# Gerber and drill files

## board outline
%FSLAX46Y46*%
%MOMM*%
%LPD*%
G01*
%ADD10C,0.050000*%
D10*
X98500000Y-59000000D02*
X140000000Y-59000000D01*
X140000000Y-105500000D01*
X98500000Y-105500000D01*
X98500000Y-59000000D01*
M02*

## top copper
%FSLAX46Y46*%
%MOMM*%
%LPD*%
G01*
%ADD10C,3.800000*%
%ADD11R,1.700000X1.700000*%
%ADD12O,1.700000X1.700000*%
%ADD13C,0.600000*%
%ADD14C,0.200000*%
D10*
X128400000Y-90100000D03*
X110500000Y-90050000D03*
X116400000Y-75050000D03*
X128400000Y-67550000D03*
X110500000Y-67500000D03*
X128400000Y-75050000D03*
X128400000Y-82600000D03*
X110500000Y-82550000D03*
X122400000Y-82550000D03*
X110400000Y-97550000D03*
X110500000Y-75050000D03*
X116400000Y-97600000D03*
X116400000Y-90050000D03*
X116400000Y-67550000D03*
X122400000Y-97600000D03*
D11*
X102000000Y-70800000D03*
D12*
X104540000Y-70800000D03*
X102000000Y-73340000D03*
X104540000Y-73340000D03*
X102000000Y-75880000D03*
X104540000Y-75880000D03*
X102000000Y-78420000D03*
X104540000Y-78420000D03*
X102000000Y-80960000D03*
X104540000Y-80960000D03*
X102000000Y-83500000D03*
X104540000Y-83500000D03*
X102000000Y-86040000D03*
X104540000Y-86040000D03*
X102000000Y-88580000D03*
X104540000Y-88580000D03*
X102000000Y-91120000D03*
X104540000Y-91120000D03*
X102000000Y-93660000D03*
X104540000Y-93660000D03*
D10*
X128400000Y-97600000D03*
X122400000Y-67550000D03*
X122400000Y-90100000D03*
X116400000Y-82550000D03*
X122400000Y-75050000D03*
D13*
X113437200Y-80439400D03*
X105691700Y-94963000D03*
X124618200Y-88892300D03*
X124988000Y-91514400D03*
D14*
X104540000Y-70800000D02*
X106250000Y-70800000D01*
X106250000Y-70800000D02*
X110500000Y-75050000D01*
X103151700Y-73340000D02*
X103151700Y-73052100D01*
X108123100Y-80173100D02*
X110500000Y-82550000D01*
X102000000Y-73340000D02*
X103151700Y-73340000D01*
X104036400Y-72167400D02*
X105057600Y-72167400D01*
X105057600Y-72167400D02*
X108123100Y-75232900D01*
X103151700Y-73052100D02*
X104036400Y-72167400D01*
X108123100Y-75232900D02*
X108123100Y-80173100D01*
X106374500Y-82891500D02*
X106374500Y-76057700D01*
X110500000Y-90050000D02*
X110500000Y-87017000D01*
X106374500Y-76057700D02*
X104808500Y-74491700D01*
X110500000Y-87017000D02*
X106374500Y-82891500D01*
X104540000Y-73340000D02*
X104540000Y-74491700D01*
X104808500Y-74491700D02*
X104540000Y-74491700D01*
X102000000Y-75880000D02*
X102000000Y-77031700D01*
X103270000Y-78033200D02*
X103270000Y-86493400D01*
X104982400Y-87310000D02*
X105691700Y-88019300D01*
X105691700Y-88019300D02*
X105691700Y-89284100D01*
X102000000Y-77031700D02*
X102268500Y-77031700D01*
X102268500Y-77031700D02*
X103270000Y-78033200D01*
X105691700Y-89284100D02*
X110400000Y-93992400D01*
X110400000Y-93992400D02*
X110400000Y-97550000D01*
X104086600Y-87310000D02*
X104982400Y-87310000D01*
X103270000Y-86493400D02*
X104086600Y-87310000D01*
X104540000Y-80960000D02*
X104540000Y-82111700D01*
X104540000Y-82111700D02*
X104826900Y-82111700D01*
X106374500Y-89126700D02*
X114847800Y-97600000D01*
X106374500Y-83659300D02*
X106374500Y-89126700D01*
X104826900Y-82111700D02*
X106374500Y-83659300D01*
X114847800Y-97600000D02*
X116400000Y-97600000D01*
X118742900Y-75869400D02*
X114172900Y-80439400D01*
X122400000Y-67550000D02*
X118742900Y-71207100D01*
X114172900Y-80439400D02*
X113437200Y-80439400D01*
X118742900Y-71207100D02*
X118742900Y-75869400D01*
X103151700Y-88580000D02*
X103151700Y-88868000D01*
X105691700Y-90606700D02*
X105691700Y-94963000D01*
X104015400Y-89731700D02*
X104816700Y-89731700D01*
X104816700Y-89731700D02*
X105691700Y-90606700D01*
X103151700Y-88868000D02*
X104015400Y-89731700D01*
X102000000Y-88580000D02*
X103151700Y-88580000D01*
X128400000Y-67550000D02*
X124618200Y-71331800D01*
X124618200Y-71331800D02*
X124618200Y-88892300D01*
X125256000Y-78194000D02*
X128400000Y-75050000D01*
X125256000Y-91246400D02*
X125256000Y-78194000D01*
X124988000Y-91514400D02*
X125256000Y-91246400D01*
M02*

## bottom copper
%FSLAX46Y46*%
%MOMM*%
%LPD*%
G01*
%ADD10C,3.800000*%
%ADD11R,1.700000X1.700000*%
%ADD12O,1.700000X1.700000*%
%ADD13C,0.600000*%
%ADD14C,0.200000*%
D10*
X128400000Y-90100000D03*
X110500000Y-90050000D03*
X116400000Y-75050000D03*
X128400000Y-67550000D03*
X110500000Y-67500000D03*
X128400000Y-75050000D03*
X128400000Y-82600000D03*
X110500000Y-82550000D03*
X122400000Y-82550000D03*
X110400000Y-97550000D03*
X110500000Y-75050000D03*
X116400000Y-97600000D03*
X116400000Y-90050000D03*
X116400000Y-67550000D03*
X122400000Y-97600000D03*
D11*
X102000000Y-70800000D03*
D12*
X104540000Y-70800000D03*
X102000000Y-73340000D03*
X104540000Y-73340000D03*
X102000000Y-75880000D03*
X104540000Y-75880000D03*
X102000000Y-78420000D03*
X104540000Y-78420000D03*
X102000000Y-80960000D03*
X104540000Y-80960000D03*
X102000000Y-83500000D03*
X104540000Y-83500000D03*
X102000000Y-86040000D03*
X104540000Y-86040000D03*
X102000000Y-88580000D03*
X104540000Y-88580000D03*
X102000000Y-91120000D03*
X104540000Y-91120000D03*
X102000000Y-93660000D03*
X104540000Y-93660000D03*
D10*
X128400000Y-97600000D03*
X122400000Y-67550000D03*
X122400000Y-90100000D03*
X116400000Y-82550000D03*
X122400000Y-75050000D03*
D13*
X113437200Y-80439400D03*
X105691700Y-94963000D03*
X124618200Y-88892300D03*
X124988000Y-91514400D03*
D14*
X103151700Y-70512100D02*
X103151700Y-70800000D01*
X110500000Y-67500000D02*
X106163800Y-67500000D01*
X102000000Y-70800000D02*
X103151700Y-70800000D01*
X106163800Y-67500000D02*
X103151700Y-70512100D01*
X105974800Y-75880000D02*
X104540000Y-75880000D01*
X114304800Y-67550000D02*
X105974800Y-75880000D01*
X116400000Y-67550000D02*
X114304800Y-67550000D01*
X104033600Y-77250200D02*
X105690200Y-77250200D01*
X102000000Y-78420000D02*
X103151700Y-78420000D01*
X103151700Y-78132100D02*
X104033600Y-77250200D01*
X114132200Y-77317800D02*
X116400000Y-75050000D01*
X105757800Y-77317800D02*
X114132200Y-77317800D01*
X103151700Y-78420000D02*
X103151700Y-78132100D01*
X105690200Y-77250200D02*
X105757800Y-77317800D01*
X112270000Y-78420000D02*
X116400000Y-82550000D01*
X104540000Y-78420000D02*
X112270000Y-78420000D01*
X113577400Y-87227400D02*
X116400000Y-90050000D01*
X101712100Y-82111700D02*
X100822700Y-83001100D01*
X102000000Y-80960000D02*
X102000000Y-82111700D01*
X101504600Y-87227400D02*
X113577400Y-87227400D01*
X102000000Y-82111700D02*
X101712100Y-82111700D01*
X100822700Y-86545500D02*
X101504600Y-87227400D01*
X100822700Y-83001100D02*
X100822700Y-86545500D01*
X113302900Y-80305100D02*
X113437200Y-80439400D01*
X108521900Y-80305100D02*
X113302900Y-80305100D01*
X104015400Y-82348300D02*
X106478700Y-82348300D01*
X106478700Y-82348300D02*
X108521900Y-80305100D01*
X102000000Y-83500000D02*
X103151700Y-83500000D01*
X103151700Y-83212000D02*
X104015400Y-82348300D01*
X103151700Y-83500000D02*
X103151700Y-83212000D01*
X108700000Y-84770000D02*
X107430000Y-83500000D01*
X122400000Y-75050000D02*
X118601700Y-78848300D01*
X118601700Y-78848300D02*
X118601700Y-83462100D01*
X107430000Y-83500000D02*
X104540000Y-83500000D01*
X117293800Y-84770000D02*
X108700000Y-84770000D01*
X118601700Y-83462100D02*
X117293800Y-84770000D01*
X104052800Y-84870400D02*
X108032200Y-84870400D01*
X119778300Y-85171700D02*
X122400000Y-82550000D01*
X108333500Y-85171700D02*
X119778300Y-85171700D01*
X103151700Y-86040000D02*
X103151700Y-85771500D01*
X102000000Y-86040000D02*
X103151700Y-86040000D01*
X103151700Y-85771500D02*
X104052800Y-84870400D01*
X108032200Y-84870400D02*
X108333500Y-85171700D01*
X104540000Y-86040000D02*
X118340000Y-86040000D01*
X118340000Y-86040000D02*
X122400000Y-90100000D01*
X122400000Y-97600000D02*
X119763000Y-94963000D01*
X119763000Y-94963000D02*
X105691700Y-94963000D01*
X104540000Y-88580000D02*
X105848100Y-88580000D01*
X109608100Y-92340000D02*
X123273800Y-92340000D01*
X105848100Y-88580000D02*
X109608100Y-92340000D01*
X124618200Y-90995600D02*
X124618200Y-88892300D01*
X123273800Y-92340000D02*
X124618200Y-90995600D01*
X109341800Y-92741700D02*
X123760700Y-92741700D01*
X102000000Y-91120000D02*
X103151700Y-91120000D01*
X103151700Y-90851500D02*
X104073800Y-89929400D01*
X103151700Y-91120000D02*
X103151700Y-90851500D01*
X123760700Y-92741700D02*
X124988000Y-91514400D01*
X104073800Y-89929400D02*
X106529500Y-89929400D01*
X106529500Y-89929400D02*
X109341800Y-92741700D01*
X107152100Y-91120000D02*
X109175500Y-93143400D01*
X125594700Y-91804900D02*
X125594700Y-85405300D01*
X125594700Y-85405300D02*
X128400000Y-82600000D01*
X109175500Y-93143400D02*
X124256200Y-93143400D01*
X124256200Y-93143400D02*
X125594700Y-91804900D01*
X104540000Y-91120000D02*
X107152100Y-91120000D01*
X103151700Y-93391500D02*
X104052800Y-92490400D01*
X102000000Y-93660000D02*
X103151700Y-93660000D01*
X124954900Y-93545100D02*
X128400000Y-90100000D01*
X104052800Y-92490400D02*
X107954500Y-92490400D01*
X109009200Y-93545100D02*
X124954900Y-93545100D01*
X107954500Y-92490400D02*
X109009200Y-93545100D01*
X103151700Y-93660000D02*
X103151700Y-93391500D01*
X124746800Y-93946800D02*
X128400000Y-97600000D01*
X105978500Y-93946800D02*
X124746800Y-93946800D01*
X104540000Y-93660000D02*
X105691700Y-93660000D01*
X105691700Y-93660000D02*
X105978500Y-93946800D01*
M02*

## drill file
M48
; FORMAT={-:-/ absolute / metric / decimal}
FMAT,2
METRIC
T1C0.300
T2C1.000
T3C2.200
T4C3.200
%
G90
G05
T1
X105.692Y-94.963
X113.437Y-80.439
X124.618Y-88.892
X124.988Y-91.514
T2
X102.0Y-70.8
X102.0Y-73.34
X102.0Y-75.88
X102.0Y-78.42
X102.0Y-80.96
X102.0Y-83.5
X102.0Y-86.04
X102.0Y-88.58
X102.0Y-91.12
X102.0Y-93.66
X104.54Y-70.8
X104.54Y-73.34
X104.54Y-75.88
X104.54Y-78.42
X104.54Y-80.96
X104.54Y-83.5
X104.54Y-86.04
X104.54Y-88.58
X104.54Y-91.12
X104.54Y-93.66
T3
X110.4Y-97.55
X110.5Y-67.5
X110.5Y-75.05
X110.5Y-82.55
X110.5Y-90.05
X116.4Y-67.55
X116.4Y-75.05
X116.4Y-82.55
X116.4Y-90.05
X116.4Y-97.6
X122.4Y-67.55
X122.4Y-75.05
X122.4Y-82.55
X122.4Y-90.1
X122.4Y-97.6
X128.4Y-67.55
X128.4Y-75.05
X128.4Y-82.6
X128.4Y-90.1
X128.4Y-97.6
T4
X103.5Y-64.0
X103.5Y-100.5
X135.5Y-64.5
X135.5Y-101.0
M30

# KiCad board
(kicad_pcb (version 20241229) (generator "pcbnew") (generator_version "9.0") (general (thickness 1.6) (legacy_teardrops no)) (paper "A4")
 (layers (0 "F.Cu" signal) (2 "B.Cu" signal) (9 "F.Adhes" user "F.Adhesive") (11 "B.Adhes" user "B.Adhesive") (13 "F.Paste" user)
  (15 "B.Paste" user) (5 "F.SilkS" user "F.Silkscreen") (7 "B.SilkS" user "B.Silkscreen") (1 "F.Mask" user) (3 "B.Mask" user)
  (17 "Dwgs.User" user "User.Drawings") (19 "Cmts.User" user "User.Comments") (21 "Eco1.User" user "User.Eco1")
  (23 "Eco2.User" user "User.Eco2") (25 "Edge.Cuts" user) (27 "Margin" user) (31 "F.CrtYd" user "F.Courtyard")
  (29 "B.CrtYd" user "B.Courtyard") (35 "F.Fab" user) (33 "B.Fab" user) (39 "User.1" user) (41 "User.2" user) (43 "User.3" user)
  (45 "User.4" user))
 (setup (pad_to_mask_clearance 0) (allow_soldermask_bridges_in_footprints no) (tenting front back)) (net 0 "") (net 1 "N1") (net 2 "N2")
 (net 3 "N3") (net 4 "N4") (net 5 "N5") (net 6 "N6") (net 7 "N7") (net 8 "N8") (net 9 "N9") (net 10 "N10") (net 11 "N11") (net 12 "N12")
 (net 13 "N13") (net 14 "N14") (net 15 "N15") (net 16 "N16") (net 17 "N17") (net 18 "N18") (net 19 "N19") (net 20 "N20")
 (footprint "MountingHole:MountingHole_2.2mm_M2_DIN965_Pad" (layer "F.Cu") (at 128.4 90.1)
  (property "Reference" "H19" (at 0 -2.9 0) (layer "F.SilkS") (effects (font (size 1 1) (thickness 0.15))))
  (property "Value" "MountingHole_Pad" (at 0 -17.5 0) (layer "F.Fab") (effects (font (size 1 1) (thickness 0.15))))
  (pad "1" thru_hole circle (at 0 0) (size 3.8 3.8) (drill 2.2) (layers "*.Cu" "*.Mask") (remove_unused_layers no) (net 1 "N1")))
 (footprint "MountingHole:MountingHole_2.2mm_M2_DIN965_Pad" (layer "F.Cu") (at 110.5 90.05)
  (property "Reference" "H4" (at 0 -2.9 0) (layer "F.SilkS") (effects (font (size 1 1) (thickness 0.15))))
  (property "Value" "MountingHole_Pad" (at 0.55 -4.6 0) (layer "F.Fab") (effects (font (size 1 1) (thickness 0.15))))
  (pad "1" thru_hole circle (at 0 0) (size 3.8 3.8) (drill 2.2) (layers "*.Cu" "*.Mask") (remove_unused_layers no) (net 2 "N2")))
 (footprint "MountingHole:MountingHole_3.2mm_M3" (layer "F.Cu") (at 135.5 64.5)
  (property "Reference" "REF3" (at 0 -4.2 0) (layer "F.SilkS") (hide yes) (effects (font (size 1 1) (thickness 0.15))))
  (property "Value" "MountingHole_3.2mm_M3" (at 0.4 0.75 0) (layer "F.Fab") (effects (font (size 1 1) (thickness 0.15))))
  (pad "" np_thru_hole circle (at 0 0) (size 3.2 3.2) (drill 3.2) (layers "*.Cu" "*.Mask")))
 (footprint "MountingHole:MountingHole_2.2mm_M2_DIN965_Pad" (layer "F.Cu") (at 116.4 75.05)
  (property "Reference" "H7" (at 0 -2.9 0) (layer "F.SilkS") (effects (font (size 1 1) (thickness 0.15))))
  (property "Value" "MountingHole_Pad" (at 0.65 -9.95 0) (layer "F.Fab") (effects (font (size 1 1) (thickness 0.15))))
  (pad "1" thru_hole circle (at 0 0) (size 3.8 3.8) (drill 2.2) (layers "*.Cu" "*.Mask") (remove_unused_layers no) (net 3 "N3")))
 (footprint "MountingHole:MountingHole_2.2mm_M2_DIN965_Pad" (layer "F.Cu") (at 128.4 67.55)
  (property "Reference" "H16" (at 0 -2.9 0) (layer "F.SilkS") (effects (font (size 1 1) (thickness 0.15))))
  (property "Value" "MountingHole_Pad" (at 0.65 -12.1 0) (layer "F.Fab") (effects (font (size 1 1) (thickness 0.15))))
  (pad "1" thru_hole circle (at 0 0) (size 3.8 3.8) (drill 2.2) (layers "*.Cu" "*.Mask") (remove_unused_layers no) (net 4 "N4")))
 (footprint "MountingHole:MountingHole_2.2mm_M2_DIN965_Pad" (layer "F.Cu") (at 110.5 67.5)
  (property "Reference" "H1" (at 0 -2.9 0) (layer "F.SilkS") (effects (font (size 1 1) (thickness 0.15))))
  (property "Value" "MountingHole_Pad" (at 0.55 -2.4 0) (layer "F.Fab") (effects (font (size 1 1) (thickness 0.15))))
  (pad "1" thru_hole circle (at 0 0) (size 3.8 3.8) (drill 2.2) (layers "*.Cu" "*.Mask") (remove_unused_layers no) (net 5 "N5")))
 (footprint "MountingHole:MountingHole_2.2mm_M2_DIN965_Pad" (layer "F.Cu") (at 128.4 75.05)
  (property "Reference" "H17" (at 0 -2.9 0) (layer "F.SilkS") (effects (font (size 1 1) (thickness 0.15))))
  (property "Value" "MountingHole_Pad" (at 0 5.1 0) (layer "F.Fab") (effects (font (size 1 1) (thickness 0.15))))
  (pad "1" thru_hole circle (at 0 0) (size 3.8 3.8) (drill 2.2) (layers "*.Cu" "*.Mask") (remove_unused_layers no) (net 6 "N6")))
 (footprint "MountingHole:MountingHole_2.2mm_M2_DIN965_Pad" (layer "F.Cu") (at 128.4 82.6)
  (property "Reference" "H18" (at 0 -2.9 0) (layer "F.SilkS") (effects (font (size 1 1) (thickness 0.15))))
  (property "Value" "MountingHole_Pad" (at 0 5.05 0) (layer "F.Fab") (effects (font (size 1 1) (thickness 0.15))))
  (pad "1" thru_hole circle (at 0 0) (size 3.8 3.8) (drill 2.2) (layers "*.Cu" "*.Mask") (remove_unused_layers no) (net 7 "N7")))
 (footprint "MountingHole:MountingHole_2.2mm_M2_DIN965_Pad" (layer "F.Cu") (at 110.5 82.55)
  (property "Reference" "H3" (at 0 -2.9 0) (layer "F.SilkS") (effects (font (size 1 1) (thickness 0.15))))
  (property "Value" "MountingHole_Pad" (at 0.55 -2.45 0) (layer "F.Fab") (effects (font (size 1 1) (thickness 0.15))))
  (pad "1" thru_hole circle (at 0 0) (size 3.8 3.8) (drill 2.2) (layers "*.Cu" "*.Mask") (remove_unused_layers no) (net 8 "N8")))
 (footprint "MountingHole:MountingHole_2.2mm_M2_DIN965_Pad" (layer "F.Cu") (at 122.4 82.55)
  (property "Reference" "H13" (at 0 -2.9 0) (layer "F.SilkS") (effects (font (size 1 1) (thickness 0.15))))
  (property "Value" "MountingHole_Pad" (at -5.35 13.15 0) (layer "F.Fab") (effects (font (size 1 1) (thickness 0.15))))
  (pad "1" thru_hole circle (at 0 0) (size 3.8 3.8) (drill 2.2) (layers "*.Cu" "*.Mask") (remove_unused_layers no) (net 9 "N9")))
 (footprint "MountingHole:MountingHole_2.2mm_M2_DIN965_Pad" (layer "F.Cu") (at 110.4 97.55)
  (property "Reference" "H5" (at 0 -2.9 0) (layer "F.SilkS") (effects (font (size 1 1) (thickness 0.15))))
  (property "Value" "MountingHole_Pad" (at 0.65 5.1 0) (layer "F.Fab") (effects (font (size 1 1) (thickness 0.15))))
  (pad "1" thru_hole circle (at 0 0) (size 3.8 3.8) (drill 2.2) (layers "*.Cu" "*.Mask") (remove_unused_layers no) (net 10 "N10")))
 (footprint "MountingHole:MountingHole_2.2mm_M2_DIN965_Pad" (layer "F.Cu") (at 110.5 75.05)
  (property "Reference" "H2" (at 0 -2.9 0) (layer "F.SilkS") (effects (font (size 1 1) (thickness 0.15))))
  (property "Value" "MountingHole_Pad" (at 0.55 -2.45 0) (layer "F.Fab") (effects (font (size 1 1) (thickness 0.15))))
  (pad "1" thru_hole circle (at 0 0) (size 3.8 3.8) (drill 2.2) (layers "*.Cu" "*.Mask") (remove_unused_layers no) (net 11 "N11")))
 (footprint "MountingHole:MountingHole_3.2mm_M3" (layer "F.Cu") (at 135.5 101)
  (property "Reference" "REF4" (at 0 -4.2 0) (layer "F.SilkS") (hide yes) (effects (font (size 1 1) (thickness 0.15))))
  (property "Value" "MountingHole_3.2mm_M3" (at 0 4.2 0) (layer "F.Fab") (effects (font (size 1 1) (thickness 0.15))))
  (pad "" np_thru_hole circle (at 0 0) (size 3.2 3.2) (drill 3.2) (layers "*.Cu" "*.Mask")))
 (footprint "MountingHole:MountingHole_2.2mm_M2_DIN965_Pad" (layer "F.Cu") (at 116.4 97.6)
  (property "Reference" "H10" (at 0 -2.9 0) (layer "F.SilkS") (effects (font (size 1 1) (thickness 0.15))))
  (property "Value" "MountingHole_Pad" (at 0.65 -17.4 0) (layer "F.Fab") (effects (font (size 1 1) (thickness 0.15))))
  (pad "1" thru_hole circle (at 0 0) (size 3.8 3.8) (drill 2.2) (layers "*.Cu" "*.Mask") (remove_unused_layers no) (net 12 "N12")))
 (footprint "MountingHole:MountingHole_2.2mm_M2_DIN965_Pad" (layer "F.Cu") (at 116.4 90.05)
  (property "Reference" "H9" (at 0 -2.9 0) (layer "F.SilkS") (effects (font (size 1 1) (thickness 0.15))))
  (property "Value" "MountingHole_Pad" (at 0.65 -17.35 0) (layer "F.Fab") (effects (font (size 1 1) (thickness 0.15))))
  (pad "1" thru_hole circle (at 0 0) (size 3.8 3.8) (drill 2.2) (layers "*.Cu" "*.Mask") (remove_unused_layers no) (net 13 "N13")))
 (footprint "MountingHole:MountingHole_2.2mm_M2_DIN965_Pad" (layer "F.Cu") (at 116.4 67.55)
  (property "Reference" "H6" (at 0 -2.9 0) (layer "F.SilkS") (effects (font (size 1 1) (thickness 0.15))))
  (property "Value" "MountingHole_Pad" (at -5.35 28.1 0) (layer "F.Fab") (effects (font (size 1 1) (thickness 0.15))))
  (pad "1" thru_hole circle (at 0 0) (size 3.8 3.8) (drill 2.2) (layers "*.Cu" "*.Mask") (remove_unused_layers no) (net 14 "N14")))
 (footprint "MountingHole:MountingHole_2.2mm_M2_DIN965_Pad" (layer "F.Cu") (at 122.4 97.6)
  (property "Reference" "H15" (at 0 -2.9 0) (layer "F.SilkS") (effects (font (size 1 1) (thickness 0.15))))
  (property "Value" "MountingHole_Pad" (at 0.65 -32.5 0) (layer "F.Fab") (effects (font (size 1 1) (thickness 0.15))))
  (pad "1" thru_hole circle (at 0 0) (size 3.8 3.8) (drill 2.2) (layers "*.Cu" "*.Mask") (remove_unused_layers no) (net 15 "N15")))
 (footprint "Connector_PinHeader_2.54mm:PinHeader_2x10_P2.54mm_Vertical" (layer "F.Cu") (at 102 70.8)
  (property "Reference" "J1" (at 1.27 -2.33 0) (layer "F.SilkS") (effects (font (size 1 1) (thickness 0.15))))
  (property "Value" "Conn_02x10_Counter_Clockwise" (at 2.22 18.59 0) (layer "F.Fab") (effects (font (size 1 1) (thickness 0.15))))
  (pad "1" thru_hole rect (at 0 0) (size 1.7 1.7) (drill 1) (layers "*.Cu" "*.Mask") (remove_unused_layers no) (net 5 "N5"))
  (pad "2" thru_hole oval (at 2.54 0) (size 1.7 1.7) (drill 1) (layers "*.Cu" "*.Mask") (remove_unused_layers no) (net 11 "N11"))
  (pad "3" thru_hole oval (at 0 2.54) (size 1.7 1.7) (drill 1) (layers "*.Cu" "*.Mask") (remove_unused_layers no) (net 8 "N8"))
  (pad "4" thru_hole oval (at 2.54 2.54) (size 1.7 1.7) (drill 1) (layers "*.Cu" "*.Mask") (remove_unused_layers no) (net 2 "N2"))
  (pad "5" thru_hole oval (at 0 5.08) (size 1.7 1.7) (drill 1) (layers "*.Cu" "*.Mask") (remove_unused_layers no) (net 10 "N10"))
  (pad "6" thru_hole oval (at 2.54 5.08) (size 1.7 1.7) (drill 1) (layers "*.Cu" "*.Mask") (remove_unused_layers no) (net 14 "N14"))
  (pad "7" thru_hole oval (at 0 7.62) (size 1.7 1.7) (drill 1) (layers "*.Cu" "*.Mask") (remove_unused_layers no) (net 3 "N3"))
  (pad "8" thru_hole oval (at 2.54 7.62) (size 1.7 1.7) (drill 1) (layers "*.Cu" "*.Mask") (remove_unused_layers no) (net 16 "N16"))
  (pad "9" thru_hole oval (at 0 10.16) (size 1.7 1.7) (drill 1) (layers "*.Cu" "*.Mask") (remove_unused_layers no) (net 13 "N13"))
  (pad "10" thru_hole oval (at 2.54 10.16) (size 1.7 1.7) (drill 1) (layers "*.Cu" "*.Mask") (remove_unused_layers no) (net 12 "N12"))
  (pad "11" thru_hole oval (at 0 12.7) (size 1.7 1.7) (drill 1) (layers "*.Cu" "*.Mask") (remove_unused_layers no) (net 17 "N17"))
  (pad "12" thru_hole oval (at 2.54 12.7) (size 1.7 1.7) (drill 1) (layers "*.Cu" "*.Mask") (remove_unused_layers no) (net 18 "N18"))
  (pad "13" thru_hole oval (at 0 15.24) (size 1.7 1.7) (drill 1) (layers "*.Cu" "*.Mask") (remove_unused_layers no) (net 9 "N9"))
  (pad "14" thru_hole oval (at 2.54 15.24) (size 1.7 1.7) (drill 1) (layers "*.Cu" "*.Mask") (remove_unused_layers no) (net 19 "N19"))
  (pad "15" thru_hole oval (at 0 17.78) (size 1.7 1.7) (drill 1) (layers "*.Cu" "*.Mask") (remove_unused_layers no) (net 15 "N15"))
  (pad "16" thru_hole oval (at 2.54 17.78) (size 1.7 1.7) (drill 1) (layers "*.Cu" "*.Mask") (remove_unused_layers no) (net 4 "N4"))
  (pad "17" thru_hole oval (at 0 20.32) (size 1.7 1.7) (drill 1) (layers "*.Cu" "*.Mask") (remove_unused_layers no) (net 6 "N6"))
  (pad "18" thru_hole oval (at 2.54 20.32) (size 1.7 1.7) (drill 1) (layers "*.Cu" "*.Mask") (remove_unused_layers no) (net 7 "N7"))
  (pad "19" thru_hole oval (at 0 22.86) (size 1.7 1.7) (drill 1) (layers "*.Cu" "*.Mask") (remove_unused_layers no) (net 1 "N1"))
  (pad "20" thru_hole oval (at 2.54 22.86) (size 1.7 1.7) (drill 1) (layers "*.Cu" "*.Mask") (remove_unused_layers no) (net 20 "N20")))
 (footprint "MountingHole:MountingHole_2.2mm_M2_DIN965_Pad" (layer "F.Cu") (at 128.4 97.6)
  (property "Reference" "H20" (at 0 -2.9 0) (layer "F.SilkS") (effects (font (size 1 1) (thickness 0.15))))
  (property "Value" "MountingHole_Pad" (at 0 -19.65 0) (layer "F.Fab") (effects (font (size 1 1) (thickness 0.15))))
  (pad "1" thru_hole circle (at 0 0) (size 3.8 3.8) (drill 2.2) (layers "*.Cu" "*.Mask") (remove_unused_layers no) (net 20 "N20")))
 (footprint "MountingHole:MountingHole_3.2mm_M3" (layer "F.Cu") (at 103.5 100.5)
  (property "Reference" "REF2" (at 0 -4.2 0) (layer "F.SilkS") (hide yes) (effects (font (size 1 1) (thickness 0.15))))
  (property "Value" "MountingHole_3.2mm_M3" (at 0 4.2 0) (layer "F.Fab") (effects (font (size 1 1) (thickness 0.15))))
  (pad "" np_thru_hole circle (at 0 0) (size 3.2 3.2) (drill 3.2) (layers "*.Cu" "*.Mask")))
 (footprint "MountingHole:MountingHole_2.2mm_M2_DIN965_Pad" (layer "F.Cu") (at 122.4 67.55)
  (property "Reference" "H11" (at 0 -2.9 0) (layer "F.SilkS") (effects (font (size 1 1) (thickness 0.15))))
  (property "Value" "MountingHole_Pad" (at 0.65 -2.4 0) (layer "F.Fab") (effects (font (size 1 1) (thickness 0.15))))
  (pad "1" thru_hole circle (at 0 0) (size 3.8 3.8) (drill 2.2) (layers "*.Cu" "*.Mask") (remove_unused_layers no) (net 17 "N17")))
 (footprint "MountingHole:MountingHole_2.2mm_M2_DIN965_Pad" (layer "F.Cu") (at 122.4 90.1)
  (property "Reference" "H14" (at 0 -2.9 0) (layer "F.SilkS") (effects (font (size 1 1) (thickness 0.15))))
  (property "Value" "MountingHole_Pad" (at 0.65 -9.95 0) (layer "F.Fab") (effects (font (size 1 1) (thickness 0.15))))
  (pad "1" thru_hole circle (at 0 0) (size 3.8 3.8) (drill 2.2) (layers "*.Cu" "*.Mask") (remove_unused_layers no) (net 19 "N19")))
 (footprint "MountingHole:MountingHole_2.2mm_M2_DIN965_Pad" (layer "F.Cu") (at 116.4 82.55)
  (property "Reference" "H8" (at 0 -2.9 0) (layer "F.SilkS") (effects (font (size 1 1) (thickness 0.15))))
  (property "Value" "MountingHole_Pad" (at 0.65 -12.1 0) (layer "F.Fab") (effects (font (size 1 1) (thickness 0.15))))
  (pad "1" thru_hole circle (at 0 0) (size 3.8 3.8) (drill 2.2) (layers "*.Cu" "*.Mask") (remove_unused_layers no) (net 16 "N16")))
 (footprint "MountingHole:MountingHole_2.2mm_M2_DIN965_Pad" (layer "F.Cu") (at 122.4 75.05)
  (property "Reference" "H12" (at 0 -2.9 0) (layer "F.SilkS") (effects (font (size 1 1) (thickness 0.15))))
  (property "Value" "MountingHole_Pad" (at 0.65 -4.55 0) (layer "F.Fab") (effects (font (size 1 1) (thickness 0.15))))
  (pad "1" thru_hole circle (at 0 0) (size 3.8 3.8) (drill 2.2) (layers "*.Cu" "*.Mask") (remove_unused_layers no) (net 18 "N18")))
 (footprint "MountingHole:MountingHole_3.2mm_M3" (layer "F.Cu") (at 103.5 64)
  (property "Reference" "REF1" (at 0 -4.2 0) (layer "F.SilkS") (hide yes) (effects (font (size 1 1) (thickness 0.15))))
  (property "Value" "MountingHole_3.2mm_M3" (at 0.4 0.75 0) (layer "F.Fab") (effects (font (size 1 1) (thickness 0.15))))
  (pad "" np_thru_hole circle (at 0 0) (size 3.2 3.2) (drill 3.2) (layers "*.Cu" "*.Mask")))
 (gr_rect (start 98.5 59) (end 140 105.5) (stroke (width 0.05) (type default)) (fill no) (layer "Edge.Cuts"))
 (segment (start 103.1517 70.5121) (end 103.1517 70.8) (width 0.2) (layer "B.Cu") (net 5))
 (segment (start 110.5 67.5) (end 106.1638 67.5) (width 0.2) (layer "B.Cu") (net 5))
 (segment (start 102 70.8) (end 103.1517 70.8) (width 0.2) (layer "B.Cu") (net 5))
 (segment (start 106.1638 67.5) (end 103.1517 70.5121) (width 0.2) (layer "B.Cu") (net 5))
 (segment (start 104.54 70.8) (end 106.25 70.8) (width 0.2) (layer "F.Cu") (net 11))
 (segment (start 106.25 70.8) (end 110.5 75.05) (width 0.2) (layer "F.Cu") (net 11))
 (segment (start 103.1517 73.34) (end 103.1517 73.0521) (width 0.2) (layer "F.Cu") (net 8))
 (segment (start 108.1231 80.1731) (end 110.5 82.55) (width 0.2) (layer "F.Cu") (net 8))
 (segment (start 102 73.34) (end 103.1517 73.34) (width 0.2) (layer "F.Cu") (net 8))
 (segment (start 104.0364 72.1674) (end 105.0576 72.1674) (width 0.2) (layer "F.Cu") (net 8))
 (segment (start 105.0576 72.1674) (end 108.1231 75.2329) (width 0.2) (layer "F.Cu") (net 8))
 (segment (start 103.1517 73.0521) (end 104.0364 72.1674) (width 0.2) (layer "F.Cu") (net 8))
 (segment (start 108.1231 75.2329) (end 108.1231 80.1731) (width 0.2) (layer "F.Cu") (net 8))
 (segment (start 106.3745 82.8915) (end 106.3745 76.0577) (width 0.2) (layer "F.Cu") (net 2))
 (segment (start 110.5 90.05) (end 110.5 87.017) (width 0.2) (layer "F.Cu") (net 2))
 (segment (start 106.3745 76.0577) (end 104.8085 74.4917) (width 0.2) (layer "F.Cu") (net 2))
 (segment (start 110.5 87.017) (end 106.3745 82.8915) (width 0.2) (layer "F.Cu") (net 2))
 (segment (start 104.54 73.34) (end 104.54 74.4917) (width 0.2) (layer "F.Cu") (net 2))
 (segment (start 104.8085 74.4917) (end 104.54 74.4917) (width 0.2) (layer "F.Cu") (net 2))
 (segment (start 102 75.88) (end 102 77.0317) (width 0.2) (layer "F.Cu") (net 10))
 (segment (start 103.27 78.0332) (end 103.27 86.4934) (width 0.2) (layer "F.Cu") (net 10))
 (segment (start 104.9824 87.31) (end 105.6917 88.0193) (width 0.2) (layer "F.Cu") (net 10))
 (segment (start 105.6917 88.0193) (end 105.6917 89.2841) (width 0.2) (layer "F.Cu") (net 10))
 (segment (start 102 77.0317) (end 102.2685 77.0317) (width 0.2) (layer "F.Cu") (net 10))
 (segment (start 102.2685 77.0317) (end 103.27 78.0332) (width 0.2) (layer "F.Cu") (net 10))
 (segment (start 105.6917 89.2841) (end 110.4 93.9924) (width 0.2) (layer "F.Cu") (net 10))
 (segment (start 110.4 93.9924) (end 110.4 97.55) (width 0.2) (layer "F.Cu") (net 10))
 (segment (start 104.0866 87.31) (end 104.9824 87.31) (width 0.2) (layer "F.Cu") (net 10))
 (segment (start 103.27 86.4934) (end 104.0866 87.31) (width 0.2) (layer "F.Cu") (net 10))
 (segment (start 105.9748 75.88) (end 104.54 75.88) (width 0.2) (layer "B.Cu") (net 14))
 (segment (start 114.3048 67.55) (end 105.9748 75.88) (width 0.2) (layer "B.Cu") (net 14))
 (segment (start 116.4 67.55) (end 114.3048 67.55) (width 0.2) (layer "B.Cu") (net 14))
 (segment (start 104.0336 77.2502) (end 105.6902 77.2502) (width 0.2) (layer "B.Cu") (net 3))
 (segment (start 102 78.42) (end 103.1517 78.42) (width 0.2) (layer "B.Cu") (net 3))
 (segment (start 103.1517 78.1321) (end 104.0336 77.2502) (width 0.2) (layer "B.Cu") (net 3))
 (segment (start 114.1322 77.3178) (end 116.4 75.05) (width 0.2) (layer "B.Cu") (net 3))
 (segment (start 105.7578 77.3178) (end 114.1322 77.3178) (width 0.2) (layer "B.Cu") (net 3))
 (segment (start 103.1517 78.42) (end 103.1517 78.1321) (width 0.2) (layer "B.Cu") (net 3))
 (segment (start 105.6902 77.2502) (end 105.7578 77.3178) (width 0.2) (layer "B.Cu") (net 3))
 (segment (start 112.27 78.42) (end 116.4 82.55) (width 0.2) (layer "B.Cu") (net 16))
 (segment (start 104.54 78.42) (end 112.27 78.42) (width 0.2) (layer "B.Cu") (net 16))
 (segment (start 113.5774 87.2274) (end 116.4 90.05) (width 0.2) (layer "B.Cu") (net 13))
 (segment (start 101.7121 82.1117) (end 100.8227 83.0011) (width 0.2) (layer "B.Cu") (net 13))
 (segment (start 102 80.96) (end 102 82.1117) (width 0.2) (layer "B.Cu") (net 13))
 (segment (start 101.5046 87.2274) (end 113.5774 87.2274) (width 0.2) (layer "B.Cu") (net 13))
 (segment (start 102 82.1117) (end 101.7121 82.1117) (width 0.2) (layer "B.Cu") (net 13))
 (segment (start 100.8227 86.5455) (end 101.5046 87.2274) (width 0.2) (layer "B.Cu") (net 13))
 (segment (start 100.8227 83.0011) (end 100.8227 86.5455) (width 0.2) (layer "B.Cu") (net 13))
 (segment (start 104.54 80.96) (end 104.54 82.1117) (width 0.2) (layer "F.Cu") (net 12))
 (segment (start 104.54 82.1117) (end 104.8269 82.1117) (width 0.2) (layer "F.Cu") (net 12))
 (segment (start 106.3745 89.1267) (end 114.8478 97.6) (width 0.2) (layer "F.Cu") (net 12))
 (segment (start 106.3745 83.6593) (end 106.3745 89.1267) (width 0.2) (layer "F.Cu") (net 12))
 (segment (start 104.8269 82.1117) (end 106.3745 83.6593) (width 0.2) (layer "F.Cu") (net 12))
 (segment (start 114.8478 97.6) (end 116.4 97.6) (width 0.2) (layer "F.Cu") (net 12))
 (segment (start 118.7429 75.8694) (end 114.1729 80.4394) (width 0.2) (layer "F.Cu") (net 17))
 (segment (start 122.4 67.55) (end 118.7429 71.2071) (width 0.2) (layer "F.Cu") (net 17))
 (segment (start 114.1729 80.4394) (end 113.4372 80.4394) (width 0.2) (layer "F.Cu") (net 17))
 (segment (start 118.7429 71.2071) (end 118.7429 75.8694) (width 0.2) (layer "F.Cu") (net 17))
 (via (at 113.4372 80.4394) (size 0.6) (drill 0.3) (layers "F.Cu" "B.Cu") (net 17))
 (segment (start 113.3029 80.3051) (end 113.4372 80.4394) (width 0.2) (layer "B.Cu") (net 17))
 (segment (start 108.5219 80.3051) (end 113.3029 80.3051) (width 0.2) (layer "B.Cu") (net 17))
 (segment (start 104.0154 82.3483) (end 106.4787 82.3483) (width 0.2) (layer "B.Cu") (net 17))
 (segment (start 106.4787 82.3483) (end 108.5219 80.3051) (width 0.2) (layer "B.Cu") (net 17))
 (segment (start 102 83.5) (end 103.1517 83.5) (width 0.2) (layer "B.Cu") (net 17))
 (segment (start 103.1517 83.212) (end 104.0154 82.3483) (width 0.2) (layer "B.Cu") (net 17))
 (segment (start 103.1517 83.5) (end 103.1517 83.212) (width 0.2) (layer "B.Cu") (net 17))
 (segment (start 108.7 84.77) (end 107.43 83.5) (width 0.2) (layer "B.Cu") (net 18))
 (segment (start 122.4 75.05) (end 118.6017 78.8483) (width 0.2) (layer "B.Cu") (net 18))
 (segment (start 118.6017 78.8483) (end 118.6017 83.4621) (width 0.2) (layer "B.Cu") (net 18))
 (segment (start 107.43 83.5) (end 104.54 83.5) (width 0.2) (layer "B.Cu") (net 18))
 (segment (start 117.2938 84.77) (end 108.7 84.77) (width 0.2) (layer "B.Cu") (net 18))
 (segment (start 118.6017 83.4621) (end 117.2938 84.77) (width 0.2) (layer "B.Cu") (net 18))
 (segment (start 104.0528 84.8704) (end 108.0322 84.8704) (width 0.2) (layer "B.Cu") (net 9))
 (segment (start 119.7783 85.1717) (end 122.4 82.55) (width 0.2) (layer "B.Cu") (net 9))
 (segment (start 108.3335 85.1717) (end 119.7783 85.1717) (width 0.2) (layer "B.Cu") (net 9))
 (segment (start 103.1517 86.04) (end 103.1517 85.7715) (width 0.2) (layer "B.Cu") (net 9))
 (segment (start 102 86.04) (end 103.1517 86.04) (width 0.2) (layer "B.Cu") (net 9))
 (segment (start 103.1517 85.7715) (end 104.0528 84.8704) (width 0.2) (layer "B.Cu") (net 9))
 (segment (start 108.0322 84.8704) (end 108.3335 85.1717) (width 0.2) (layer "B.Cu") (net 9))
 (segment (start 104.54 86.04) (end 118.34 86.04) (width 0.2) (layer "B.Cu") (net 19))
 (segment (start 118.34 86.04) (end 122.4 90.1) (width 0.2) (layer "B.Cu") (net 19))
 (segment (start 103.1517 88.58) (end 103.1517 88.868) (width 0.2) (layer "F.Cu") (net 15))
 (segment (start 105.6917 90.6067) (end 105.6917 94.963) (width 0.2) (layer "F.Cu") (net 15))
 (segment (start 104.0154 89.7317) (end 104.8167 89.7317) (width 0.2) (layer "F.Cu") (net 15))
 (segment (start 104.8167 89.7317) (end 105.6917 90.6067) (width 0.2) (layer "F.Cu") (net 15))
 (segment (start 103.1517 88.868) (end 104.0154 89.7317) (width 0.2) (layer "F.Cu") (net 15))
 (segment (start 102 88.58) (end 103.1517 88.58) (width 0.2) (layer "F.Cu") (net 15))
 (via (at 105.6917 94.963) (size 0.6) (drill 0.3) (layers "F.Cu" "B.Cu") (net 15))
 (segment (start 122.4 97.6) (end 119.763 94.963) (width 0.2) (layer "B.Cu") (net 15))
 (segment (start 119.763 94.963) (end 105.6917 94.963) (width 0.2) (layer "B.Cu") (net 15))
 (segment (start 128.4 67.55) (end 124.6182 71.3318) (width 0.2) (layer "F.Cu") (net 4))
 (segment (start 124.6182 71.3318) (end 124.6182 88.8923) (width 0.2) (layer "F.Cu") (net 4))
 (via (at 124.6182 88.8923) (size 0.6) (drill 0.3) (layers "F.Cu" "B.Cu") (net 4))
 (segment (start 104.54 88.58) (end 105.8481 88.58) (width 0.2) (layer "B.Cu") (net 4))
 (segment (start 109.6081 92.34) (end 123.2738 92.34) (width 0.2) (layer "B.Cu") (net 4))
 (segment (start 105.8481 88.58) (end 109.6081 92.34) (width 0.2) (layer "B.Cu") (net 4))
 (segment (start 124.6182 90.9956) (end 124.6182 88.8923) (width 0.2) (layer "B.Cu") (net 4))
 (segment (start 123.2738 92.34) (end 124.6182 90.9956) (width 0.2) (layer "B.Cu") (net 4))
 (segment (start 125.256 78.194) (end 128.4 75.05) (width 0.2) (layer "F.Cu") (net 6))
 (segment (start 125.256 91.2464) (end 125.256 78.194) (width 0.2) (layer "F.Cu") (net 6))
 (segment (start 124.988 91.5144) (end 125.256 91.2464) (width 0.2) (layer "F.Cu") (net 6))
 (via (at 124.988 91.5144) (size 0.6) (drill 0.3) (layers "F.Cu" "B.Cu") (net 6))
 (segment (start 109.3418 92.7417) (end 123.7607 92.7417) (width 0.2) (layer "B.Cu") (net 6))
 (segment (start 102 91.12) (end 103.1517 91.12) (width 0.2) (layer "B.Cu") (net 6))
 (segment (start 103.1517 90.8515) (end 104.0738 89.9294) (width 0.2) (layer "B.Cu") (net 6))
 (segment (start 103.1517 91.12) (end 103.1517 90.8515) (width 0.2) (layer "B.Cu") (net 6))
 (segment (start 123.7607 92.7417) (end 124.988 91.5144) (width 0.2) (layer "B.Cu") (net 6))
 (segment (start 104.0738 89.9294) (end 106.5295 89.9294) (width 0.2) (layer "B.Cu") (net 6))
 (segment (start 106.5295 89.9294) (end 109.3418 92.7417) (width 0.2) (layer "B.Cu") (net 6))
 (segment (start 107.1521 91.12) (end 109.1755 93.1434) (width 0.2) (layer "B.Cu") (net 7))
 (segment (start 125.5947 91.8049) (end 125.5947 85.4053) (width 0.2) (layer "B.Cu") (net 7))
 (segment (start 125.5947 85.4053) (end 128.4 82.6) (width 0.2) (layer "B.Cu") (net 7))
 (segment (start 109.1755 93.1434) (end 124.2562 93.1434) (width 0.2) (layer "B.Cu") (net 7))
 (segment (start 124.2562 93.1434) (end 125.5947 91.8049) (width 0.2) (layer "B.Cu") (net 7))
 (segment (start 104.54 91.12) (end 107.1521 91.12) (width 0.2) (layer "B.Cu") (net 7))
 (segment (start 103.1517 93.3915) (end 104.0528 92.4904) (width 0.2) (layer "B.Cu") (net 1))
 (segment (start 102 93.66) (end 103.1517 93.66) (width 0.2) (layer "B.Cu") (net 1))
 (segment (start 124.9549 93.5451) (end 128.4 90.1) (width 0.2) (layer "B.Cu") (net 1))
 (segment (start 104.0528 92.4904) (end 107.9545 92.4904) (width 0.2) (layer "B.Cu") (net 1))
 (segment (start 109.0092 93.5451) (end 124.9549 93.5451) (width 0.2) (layer "B.Cu") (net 1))
 (segment (start 107.9545 92.4904) (end 109.0092 93.5451) (width 0.2) (layer "B.Cu") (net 1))
 (segment (start 103.1517 93.66) (end 103.1517 93.3915) (width 0.2) (layer "B.Cu") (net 1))
 (segment (start 124.7468 93.9468) (end 128.4 97.6) (width 0.2) (layer "B.Cu") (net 20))
 (segment (start 105.9785 93.9468) (end 124.7468 93.9468) (width 0.2) (layer "B.Cu") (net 20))
 (segment (start 104.54 93.66) (end 105.6917 93.66) (width 0.2) (layer "B.Cu") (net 20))
 (segment (start 105.6917 93.66) (end 105.9785 93.9468) (width 0.2) (layer "B.Cu") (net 20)))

